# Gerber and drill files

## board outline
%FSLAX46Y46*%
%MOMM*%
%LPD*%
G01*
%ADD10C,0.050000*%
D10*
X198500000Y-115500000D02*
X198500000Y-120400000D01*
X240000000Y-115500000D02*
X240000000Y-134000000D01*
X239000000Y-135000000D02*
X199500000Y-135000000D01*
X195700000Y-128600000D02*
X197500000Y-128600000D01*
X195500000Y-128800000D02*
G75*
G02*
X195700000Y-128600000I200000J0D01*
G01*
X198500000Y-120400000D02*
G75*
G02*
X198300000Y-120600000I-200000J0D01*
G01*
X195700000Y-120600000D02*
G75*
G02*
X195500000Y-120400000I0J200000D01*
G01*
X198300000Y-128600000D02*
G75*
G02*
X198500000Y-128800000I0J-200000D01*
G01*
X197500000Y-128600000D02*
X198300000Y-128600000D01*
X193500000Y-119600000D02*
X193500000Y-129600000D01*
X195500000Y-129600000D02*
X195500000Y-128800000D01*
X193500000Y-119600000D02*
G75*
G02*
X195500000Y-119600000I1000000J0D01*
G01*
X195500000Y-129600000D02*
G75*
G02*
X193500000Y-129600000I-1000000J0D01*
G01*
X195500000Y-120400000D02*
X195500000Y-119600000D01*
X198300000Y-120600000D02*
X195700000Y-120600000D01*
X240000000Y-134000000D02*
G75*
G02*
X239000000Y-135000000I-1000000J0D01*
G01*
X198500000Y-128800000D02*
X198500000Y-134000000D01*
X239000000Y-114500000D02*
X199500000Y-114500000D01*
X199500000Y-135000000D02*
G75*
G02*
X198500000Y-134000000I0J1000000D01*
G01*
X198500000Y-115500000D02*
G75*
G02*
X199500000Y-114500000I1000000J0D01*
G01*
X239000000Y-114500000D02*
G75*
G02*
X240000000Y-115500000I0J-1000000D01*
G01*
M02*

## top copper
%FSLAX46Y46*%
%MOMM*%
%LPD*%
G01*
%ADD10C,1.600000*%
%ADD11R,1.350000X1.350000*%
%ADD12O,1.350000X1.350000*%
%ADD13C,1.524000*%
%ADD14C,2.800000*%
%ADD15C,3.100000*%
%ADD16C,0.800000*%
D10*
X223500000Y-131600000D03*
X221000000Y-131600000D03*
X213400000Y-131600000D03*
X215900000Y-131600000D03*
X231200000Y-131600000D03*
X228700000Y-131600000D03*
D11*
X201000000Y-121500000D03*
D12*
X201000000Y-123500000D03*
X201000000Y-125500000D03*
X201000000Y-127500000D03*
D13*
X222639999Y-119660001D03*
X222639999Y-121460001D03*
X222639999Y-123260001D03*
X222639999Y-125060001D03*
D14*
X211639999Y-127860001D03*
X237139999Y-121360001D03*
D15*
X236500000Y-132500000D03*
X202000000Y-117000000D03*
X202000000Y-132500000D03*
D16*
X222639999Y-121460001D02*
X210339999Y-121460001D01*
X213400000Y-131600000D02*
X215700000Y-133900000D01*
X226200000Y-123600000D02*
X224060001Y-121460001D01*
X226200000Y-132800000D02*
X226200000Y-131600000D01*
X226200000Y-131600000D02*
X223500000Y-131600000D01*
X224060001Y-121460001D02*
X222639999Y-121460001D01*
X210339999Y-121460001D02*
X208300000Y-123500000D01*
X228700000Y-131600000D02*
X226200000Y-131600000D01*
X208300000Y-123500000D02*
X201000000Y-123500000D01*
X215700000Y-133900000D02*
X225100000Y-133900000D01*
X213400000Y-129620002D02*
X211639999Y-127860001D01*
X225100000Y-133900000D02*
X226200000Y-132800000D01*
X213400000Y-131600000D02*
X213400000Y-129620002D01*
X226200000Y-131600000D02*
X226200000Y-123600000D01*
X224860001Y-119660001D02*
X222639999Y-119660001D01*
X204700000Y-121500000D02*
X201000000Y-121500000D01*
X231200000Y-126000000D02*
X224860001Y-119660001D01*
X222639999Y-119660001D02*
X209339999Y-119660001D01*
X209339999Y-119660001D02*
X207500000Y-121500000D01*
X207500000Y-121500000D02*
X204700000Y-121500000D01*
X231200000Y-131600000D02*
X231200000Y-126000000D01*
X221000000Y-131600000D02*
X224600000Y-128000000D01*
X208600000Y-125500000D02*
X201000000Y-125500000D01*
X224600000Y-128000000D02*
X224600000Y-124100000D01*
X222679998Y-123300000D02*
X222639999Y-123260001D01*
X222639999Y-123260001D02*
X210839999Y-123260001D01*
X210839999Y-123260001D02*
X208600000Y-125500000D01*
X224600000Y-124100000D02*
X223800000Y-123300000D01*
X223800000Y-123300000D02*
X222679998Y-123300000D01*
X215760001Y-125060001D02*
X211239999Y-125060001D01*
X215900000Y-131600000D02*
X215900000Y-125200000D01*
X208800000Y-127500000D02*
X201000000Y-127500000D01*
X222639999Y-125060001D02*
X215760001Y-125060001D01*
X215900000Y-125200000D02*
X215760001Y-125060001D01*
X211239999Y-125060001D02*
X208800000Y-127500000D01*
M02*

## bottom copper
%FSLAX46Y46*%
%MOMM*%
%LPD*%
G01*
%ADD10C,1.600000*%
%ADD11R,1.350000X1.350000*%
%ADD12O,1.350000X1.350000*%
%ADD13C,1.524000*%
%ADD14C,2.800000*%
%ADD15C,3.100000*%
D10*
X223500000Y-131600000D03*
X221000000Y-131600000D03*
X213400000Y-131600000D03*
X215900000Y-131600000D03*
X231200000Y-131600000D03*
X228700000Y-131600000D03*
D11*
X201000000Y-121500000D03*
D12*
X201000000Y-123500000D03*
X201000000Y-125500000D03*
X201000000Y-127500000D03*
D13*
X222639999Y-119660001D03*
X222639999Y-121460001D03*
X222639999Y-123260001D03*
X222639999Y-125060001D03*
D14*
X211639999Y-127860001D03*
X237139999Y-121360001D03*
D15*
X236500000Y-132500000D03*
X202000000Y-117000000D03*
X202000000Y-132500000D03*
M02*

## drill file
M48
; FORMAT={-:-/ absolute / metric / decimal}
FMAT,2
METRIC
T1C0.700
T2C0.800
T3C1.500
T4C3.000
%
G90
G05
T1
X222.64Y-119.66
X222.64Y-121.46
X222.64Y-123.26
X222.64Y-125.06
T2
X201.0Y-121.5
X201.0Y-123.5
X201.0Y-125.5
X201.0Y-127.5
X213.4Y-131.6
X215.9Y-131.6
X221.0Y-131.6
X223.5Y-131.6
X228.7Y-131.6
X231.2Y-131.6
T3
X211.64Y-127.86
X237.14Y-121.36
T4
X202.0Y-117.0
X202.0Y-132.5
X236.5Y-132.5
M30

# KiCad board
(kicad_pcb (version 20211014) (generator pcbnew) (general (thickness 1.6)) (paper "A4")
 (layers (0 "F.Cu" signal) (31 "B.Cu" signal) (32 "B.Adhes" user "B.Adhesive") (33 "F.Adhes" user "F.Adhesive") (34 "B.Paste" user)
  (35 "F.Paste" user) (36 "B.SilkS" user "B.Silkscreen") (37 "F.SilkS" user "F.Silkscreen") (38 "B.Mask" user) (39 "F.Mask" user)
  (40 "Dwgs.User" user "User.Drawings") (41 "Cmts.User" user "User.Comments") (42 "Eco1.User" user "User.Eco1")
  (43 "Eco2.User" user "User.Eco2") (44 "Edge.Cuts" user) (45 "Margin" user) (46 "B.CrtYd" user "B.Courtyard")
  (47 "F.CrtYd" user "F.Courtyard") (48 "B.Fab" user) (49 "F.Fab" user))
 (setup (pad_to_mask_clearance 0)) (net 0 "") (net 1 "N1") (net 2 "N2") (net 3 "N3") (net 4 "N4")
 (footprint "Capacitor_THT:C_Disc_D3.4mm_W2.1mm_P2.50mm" (layer "F.Cu") (at 223.5 131.6 180)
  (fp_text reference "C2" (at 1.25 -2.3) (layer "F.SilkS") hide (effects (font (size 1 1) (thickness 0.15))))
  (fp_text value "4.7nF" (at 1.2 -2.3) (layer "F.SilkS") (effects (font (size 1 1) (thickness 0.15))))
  (pad "1" thru_hole circle locked (at 0 0 180) (size 1.6 1.6) (drill 0.8) (layers *.Cu *.Mask) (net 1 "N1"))
  (pad "2" thru_hole circle locked (at 2.5 0 180) (size 1.6 1.6) (drill 0.8) (layers *.Cu *.Mask) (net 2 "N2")))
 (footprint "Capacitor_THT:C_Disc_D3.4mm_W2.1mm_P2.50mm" (layer "F.Cu") (at 213.4 131.6)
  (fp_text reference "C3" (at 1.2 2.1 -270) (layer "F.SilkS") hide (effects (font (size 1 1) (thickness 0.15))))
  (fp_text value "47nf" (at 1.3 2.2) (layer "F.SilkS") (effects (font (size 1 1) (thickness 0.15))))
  (pad "1" thru_hole circle locked (at 0 0) (size 1.6 1.6) (drill 0.8) (layers *.Cu *.Mask) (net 1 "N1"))
  (pad "2" thru_hole circle locked (at 2.5 0) (size 1.6 1.6) (drill 0.8) (layers *.Cu *.Mask) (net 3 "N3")))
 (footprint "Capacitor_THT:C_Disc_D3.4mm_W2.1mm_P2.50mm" (layer "F.Cu") (at 231.2 131.6 180)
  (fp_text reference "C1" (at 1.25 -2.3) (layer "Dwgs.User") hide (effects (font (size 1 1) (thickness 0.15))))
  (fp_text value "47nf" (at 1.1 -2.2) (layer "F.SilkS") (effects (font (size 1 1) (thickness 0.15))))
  (pad "1" thru_hole circle locked (at 0 0 180) (size 1.6 1.6) (drill 0.8) (layers *.Cu *.Mask) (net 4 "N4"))
  (pad "2" thru_hole circle locked (at 2.5 0 180) (size 1.6 1.6) (drill 0.8) (layers *.Cu *.Mask) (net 1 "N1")))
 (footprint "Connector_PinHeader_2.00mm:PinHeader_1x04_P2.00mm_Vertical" (layer "F.Cu") (at 201 121.5)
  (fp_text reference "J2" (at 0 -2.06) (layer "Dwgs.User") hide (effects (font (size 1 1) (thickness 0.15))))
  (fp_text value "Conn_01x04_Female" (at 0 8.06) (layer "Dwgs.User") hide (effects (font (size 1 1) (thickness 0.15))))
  (pad "1" thru_hole rect locked (at 0 0) (size 1.35 1.35) (drill 0.8) (layers *.Cu *.Mask) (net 4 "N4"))
  (pad "2" thru_hole oval locked (at 0 2) (size 1.35 1.35) (drill 0.8) (layers *.Cu *.Mask) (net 1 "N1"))
  (pad "3" thru_hole oval locked (at 0 4) (size 1.35 1.35) (drill 0.8) (layers *.Cu *.Mask) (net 2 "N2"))
  (pad "4" thru_hole oval locked (at 0 6) (size 1.35 1.35) (drill 0.8) (layers *.Cu *.Mask) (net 3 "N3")))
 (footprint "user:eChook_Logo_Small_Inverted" (layer "F.Cu") (at 208.5 133)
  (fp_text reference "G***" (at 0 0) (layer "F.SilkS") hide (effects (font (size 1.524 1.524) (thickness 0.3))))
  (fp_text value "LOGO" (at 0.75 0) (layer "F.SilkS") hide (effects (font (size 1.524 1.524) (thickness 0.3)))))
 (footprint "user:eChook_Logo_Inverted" (layer "B.Cu") (at 213 121.2 180)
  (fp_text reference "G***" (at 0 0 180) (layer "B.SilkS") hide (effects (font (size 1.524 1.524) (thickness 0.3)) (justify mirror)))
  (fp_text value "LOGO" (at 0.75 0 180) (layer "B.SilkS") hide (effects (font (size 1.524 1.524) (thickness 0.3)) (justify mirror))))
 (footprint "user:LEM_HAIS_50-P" (layer "B.Cu") (at 222.639999 125.060001 180)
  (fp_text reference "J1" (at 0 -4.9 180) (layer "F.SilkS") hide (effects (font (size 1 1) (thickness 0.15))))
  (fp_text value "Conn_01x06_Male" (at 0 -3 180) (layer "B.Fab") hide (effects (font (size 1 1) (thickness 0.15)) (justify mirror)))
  (pad "1" thru_hole circle locked (at 0 5.4 180) (size 1.524 1.524) (drill 0.7) (layers *.Cu *.Mask) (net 4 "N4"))
  (pad "2" thru_hole circle locked (at 0 3.6 180) (size 1.524 1.524) (drill 0.7) (layers *.Cu *.Mask) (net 1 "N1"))
  (pad "3" thru_hole circle locked (at 0 1.8 180) (size 1.524 1.524) (drill 0.7) (layers *.Cu *.Mask) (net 2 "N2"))
  (pad "4" thru_hole circle locked (at 0 0 180) (size 1.524 1.524) (drill 0.7) (layers *.Cu *.Mask) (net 3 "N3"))
  (pad "5" thru_hole circle locked (at 11 -2.8 180) (size 2.8 2.8) (drill 1.5) (layers *.Cu *.Mask) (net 1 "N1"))
  (pad "6" thru_hole circle locked (at -14.5 3.7 180) (size 2.8 2.8) (drill 1.5) (layers *.Cu *.Mask)))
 (gr_line (start 198.5 115.5) (end 198.5 120.4) (layer "Edge.Cuts") (width 0.05))
 (gr_line (start 240 115.5) (end 240 134) (layer "Edge.Cuts") (width 0.05))
 (gr_line (start 239 135) (end 199.5 135) (layer "Edge.Cuts") (width 0.05))
 (gr_line (start 195.7 128.6) (end 197.5 128.6) (layer "Edge.Cuts") (width 0.05))
 (gr_arc (start 195.5 128.8) (mid 195.558579 128.658579) (end 195.7 128.6) (layer "Edge.Cuts") (width 0.05))
 (gr_arc (start 198.5 120.4) (mid 198.441421 120.541421) (end 198.3 120.6) (layer "Edge.Cuts") (width 0.05))
 (gr_arc (start 195.7 120.6) (mid 195.558579 120.541421) (end 195.5 120.4) (layer "Edge.Cuts") (width 0.05))
 (gr_arc (start 198.3 128.6) (mid 198.441421 128.658579) (end 198.5 128.8) (layer "Edge.Cuts") (width 0.05))
 (gr_line (start 197.5 128.6) (end 198.3 128.6) (layer "Edge.Cuts") (width 0.05))
 (gr_line (start 193.5 119.6) (end 193.5 129.6) (layer "Edge.Cuts") (width 0.05))
 (gr_line (start 195.5 129.6) (end 195.5 128.8) (layer "Edge.Cuts") (width 0.05))
 (gr_arc (start 193.5 119.6) (mid 194.5 118.6) (end 195.5 119.6) (layer "Edge.Cuts") (width 0.05))
 (gr_arc (start 195.5 129.6) (mid 194.5 130.6) (end 193.5 129.6) (layer "Edge.Cuts") (width 0.05))
 (gr_line (start 195.5 120.4) (end 195.5 119.6) (layer "Edge.Cuts") (width 0.05))
 (gr_line (start 198.3 120.6) (end 195.7 120.6) (layer "Edge.Cuts") (width 0.05))
 (gr_arc (start 240 134) (mid 239.707107 134.707107) (end 239 135) (layer "Edge.Cuts") (width 0.05))
 (gr_line (start 198.5 128.8) (end 198.5 134) (layer "Edge.Cuts") (width 0.05))
 (gr_line (start 239 114.5) (end 199.5 114.5) (layer "Edge.Cuts") (width 0.05))
 (gr_arc (start 199.5 135) (mid 198.792893 134.707107) (end 198.5 134) (layer "Edge.Cuts") (width 0.05))
 (gr_arc (start 198.5 115.5) (mid 198.792893 114.792893) (end 199.5 114.5) (layer "Edge.Cuts") (width 0.05))
 (gr_arc (start 239 114.5) (mid 239.707107 114.792893) (end 240 115.5) (layer "Edge.Cuts") (width 0.05))
 (via (at 236.5 132.5) (size 3.1) (drill 3) (layers "F.Cu" "B.Cu") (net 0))
 (via (at 202 117) (size 3.1) (drill 3) (layers "F.Cu" "B.Cu") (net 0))
 (via (at 202 132.5) (size 3.1) (drill 3) (layers "F.Cu" "B.Cu") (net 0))
 (segment (start 222.639999 121.460001) (end 210.339999 121.460001) (width 0.8) (layer "F.Cu") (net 1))
 (segment (start 213.4 131.6) (end 215.7 133.9) (width 0.8) (layer "F.Cu") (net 1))
 (segment (start 226.2 123.6) (end 224.060001 121.460001) (width 0.8) (layer "F.Cu") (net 1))
 (segment (start 226.2 132.8) (end 226.2 131.6) (width 0.8) (layer "F.Cu") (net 1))
 (segment (start 226.2 131.6) (end 223.5 131.6) (width 0.8) (layer "F.Cu") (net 1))
 (segment (start 224.060001 121.460001) (end 222.639999 121.460001) (width 0.8) (layer "F.Cu") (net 1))
 (segment (start 210.339999 121.460001) (end 208.3 123.5) (width 0.8) (layer "F.Cu") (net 1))
 (segment (start 228.7 131.6) (end 226.2 131.6) (width 0.8) (layer "F.Cu") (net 1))
 (segment (start 208.3 123.5) (end 201 123.5) (width 0.8) (layer "F.Cu") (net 1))
 (segment (start 215.7 133.9) (end 225.1 133.9) (width 0.8) (layer "F.Cu") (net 1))
 (segment (start 213.4 129.620002) (end 211.639999 127.860001) (width 0.8) (layer "F.Cu") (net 1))
 (segment (start 225.1 133.9) (end 226.2 132.8) (width 0.8) (layer "F.Cu") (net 1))
 (segment (start 213.4 131.6) (end 213.4 129.620002) (width 0.8) (layer "F.Cu") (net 1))
 (segment (start 226.2 131.6) (end 226.2 123.6) (width 0.8) (layer "F.Cu") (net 1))
 (segment (start 224.860001 119.660001) (end 222.639999 119.660001) (width 0.8) (layer "F.Cu") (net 4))
 (segment (start 204.7 121.5) (end 201 121.5) (width 0.8) (layer "F.Cu") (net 4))
 (segment (start 231.2 126) (end 224.860001 119.660001) (width 0.8) (layer "F.Cu") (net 4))
 (segment (start 222.639999 119.660001) (end 209.339999 119.660001) (width 0.8) (layer "F.Cu") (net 4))
 (segment (start 209.339999 119.660001) (end 207.5 121.5) (width 0.8) (layer "F.Cu") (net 4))
 (segment (start 207.5 121.5) (end 204.7 121.5) (width 0.8) (layer "F.Cu") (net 4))
 (segment (start 231.2 131.6) (end 231.2 126) (width 0.8) (layer "F.Cu") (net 4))
 (segment (start 221 131.6) (end 224.6 128) (width 0.8) (layer "F.Cu") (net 2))
 (segment (start 208.6 125.5) (end 201 125.5) (width 0.8) (layer "F.Cu") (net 2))
 (segment (start 224.6 128) (end 224.6 124.1) (width 0.8) (layer "F.Cu") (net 2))
 (segment (start 222.679998 123.3) (end 222.639999 123.260001) (width 0.8) (layer "F.Cu") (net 2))
 (segment (start 222.639999 123.260001) (end 210.839999 123.260001) (width 0.8) (layer "F.Cu") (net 2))
 (segment (start 210.839999 123.260001) (end 208.6 125.5) (width 0.8) (layer "F.Cu") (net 2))
 (segment (start 224.6 124.1) (end 223.8 123.3) (width 0.8) (layer "F.Cu") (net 2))
 (segment (start 223.8 123.3) (end 222.679998 123.3) (width 0.8) (layer "F.Cu") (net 2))
 (segment (start 215.760001 125.060001) (end 211.239999 125.060001) (width 0.8) (layer "F.Cu") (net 3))
 (segment (start 215.9 131.6) (end 215.9 125.2) (width 0.8) (layer "F.Cu") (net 3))
 (segment (start 208.8 127.5) (end 201 127.5) (width 0.8) (layer "F.Cu") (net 3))
 (segment (start 222.639999 125.060001) (end 215.760001 125.060001) (width 0.8) (layer "F.Cu") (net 3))
 (segment (start 215.9 125.2) (end 215.760001 125.060001) (width 0.8) (layer "F.Cu") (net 3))
 (segment (start 211.239999 125.060001) (end 208.8 127.5) (width 0.8) (layer "F.Cu") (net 3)))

